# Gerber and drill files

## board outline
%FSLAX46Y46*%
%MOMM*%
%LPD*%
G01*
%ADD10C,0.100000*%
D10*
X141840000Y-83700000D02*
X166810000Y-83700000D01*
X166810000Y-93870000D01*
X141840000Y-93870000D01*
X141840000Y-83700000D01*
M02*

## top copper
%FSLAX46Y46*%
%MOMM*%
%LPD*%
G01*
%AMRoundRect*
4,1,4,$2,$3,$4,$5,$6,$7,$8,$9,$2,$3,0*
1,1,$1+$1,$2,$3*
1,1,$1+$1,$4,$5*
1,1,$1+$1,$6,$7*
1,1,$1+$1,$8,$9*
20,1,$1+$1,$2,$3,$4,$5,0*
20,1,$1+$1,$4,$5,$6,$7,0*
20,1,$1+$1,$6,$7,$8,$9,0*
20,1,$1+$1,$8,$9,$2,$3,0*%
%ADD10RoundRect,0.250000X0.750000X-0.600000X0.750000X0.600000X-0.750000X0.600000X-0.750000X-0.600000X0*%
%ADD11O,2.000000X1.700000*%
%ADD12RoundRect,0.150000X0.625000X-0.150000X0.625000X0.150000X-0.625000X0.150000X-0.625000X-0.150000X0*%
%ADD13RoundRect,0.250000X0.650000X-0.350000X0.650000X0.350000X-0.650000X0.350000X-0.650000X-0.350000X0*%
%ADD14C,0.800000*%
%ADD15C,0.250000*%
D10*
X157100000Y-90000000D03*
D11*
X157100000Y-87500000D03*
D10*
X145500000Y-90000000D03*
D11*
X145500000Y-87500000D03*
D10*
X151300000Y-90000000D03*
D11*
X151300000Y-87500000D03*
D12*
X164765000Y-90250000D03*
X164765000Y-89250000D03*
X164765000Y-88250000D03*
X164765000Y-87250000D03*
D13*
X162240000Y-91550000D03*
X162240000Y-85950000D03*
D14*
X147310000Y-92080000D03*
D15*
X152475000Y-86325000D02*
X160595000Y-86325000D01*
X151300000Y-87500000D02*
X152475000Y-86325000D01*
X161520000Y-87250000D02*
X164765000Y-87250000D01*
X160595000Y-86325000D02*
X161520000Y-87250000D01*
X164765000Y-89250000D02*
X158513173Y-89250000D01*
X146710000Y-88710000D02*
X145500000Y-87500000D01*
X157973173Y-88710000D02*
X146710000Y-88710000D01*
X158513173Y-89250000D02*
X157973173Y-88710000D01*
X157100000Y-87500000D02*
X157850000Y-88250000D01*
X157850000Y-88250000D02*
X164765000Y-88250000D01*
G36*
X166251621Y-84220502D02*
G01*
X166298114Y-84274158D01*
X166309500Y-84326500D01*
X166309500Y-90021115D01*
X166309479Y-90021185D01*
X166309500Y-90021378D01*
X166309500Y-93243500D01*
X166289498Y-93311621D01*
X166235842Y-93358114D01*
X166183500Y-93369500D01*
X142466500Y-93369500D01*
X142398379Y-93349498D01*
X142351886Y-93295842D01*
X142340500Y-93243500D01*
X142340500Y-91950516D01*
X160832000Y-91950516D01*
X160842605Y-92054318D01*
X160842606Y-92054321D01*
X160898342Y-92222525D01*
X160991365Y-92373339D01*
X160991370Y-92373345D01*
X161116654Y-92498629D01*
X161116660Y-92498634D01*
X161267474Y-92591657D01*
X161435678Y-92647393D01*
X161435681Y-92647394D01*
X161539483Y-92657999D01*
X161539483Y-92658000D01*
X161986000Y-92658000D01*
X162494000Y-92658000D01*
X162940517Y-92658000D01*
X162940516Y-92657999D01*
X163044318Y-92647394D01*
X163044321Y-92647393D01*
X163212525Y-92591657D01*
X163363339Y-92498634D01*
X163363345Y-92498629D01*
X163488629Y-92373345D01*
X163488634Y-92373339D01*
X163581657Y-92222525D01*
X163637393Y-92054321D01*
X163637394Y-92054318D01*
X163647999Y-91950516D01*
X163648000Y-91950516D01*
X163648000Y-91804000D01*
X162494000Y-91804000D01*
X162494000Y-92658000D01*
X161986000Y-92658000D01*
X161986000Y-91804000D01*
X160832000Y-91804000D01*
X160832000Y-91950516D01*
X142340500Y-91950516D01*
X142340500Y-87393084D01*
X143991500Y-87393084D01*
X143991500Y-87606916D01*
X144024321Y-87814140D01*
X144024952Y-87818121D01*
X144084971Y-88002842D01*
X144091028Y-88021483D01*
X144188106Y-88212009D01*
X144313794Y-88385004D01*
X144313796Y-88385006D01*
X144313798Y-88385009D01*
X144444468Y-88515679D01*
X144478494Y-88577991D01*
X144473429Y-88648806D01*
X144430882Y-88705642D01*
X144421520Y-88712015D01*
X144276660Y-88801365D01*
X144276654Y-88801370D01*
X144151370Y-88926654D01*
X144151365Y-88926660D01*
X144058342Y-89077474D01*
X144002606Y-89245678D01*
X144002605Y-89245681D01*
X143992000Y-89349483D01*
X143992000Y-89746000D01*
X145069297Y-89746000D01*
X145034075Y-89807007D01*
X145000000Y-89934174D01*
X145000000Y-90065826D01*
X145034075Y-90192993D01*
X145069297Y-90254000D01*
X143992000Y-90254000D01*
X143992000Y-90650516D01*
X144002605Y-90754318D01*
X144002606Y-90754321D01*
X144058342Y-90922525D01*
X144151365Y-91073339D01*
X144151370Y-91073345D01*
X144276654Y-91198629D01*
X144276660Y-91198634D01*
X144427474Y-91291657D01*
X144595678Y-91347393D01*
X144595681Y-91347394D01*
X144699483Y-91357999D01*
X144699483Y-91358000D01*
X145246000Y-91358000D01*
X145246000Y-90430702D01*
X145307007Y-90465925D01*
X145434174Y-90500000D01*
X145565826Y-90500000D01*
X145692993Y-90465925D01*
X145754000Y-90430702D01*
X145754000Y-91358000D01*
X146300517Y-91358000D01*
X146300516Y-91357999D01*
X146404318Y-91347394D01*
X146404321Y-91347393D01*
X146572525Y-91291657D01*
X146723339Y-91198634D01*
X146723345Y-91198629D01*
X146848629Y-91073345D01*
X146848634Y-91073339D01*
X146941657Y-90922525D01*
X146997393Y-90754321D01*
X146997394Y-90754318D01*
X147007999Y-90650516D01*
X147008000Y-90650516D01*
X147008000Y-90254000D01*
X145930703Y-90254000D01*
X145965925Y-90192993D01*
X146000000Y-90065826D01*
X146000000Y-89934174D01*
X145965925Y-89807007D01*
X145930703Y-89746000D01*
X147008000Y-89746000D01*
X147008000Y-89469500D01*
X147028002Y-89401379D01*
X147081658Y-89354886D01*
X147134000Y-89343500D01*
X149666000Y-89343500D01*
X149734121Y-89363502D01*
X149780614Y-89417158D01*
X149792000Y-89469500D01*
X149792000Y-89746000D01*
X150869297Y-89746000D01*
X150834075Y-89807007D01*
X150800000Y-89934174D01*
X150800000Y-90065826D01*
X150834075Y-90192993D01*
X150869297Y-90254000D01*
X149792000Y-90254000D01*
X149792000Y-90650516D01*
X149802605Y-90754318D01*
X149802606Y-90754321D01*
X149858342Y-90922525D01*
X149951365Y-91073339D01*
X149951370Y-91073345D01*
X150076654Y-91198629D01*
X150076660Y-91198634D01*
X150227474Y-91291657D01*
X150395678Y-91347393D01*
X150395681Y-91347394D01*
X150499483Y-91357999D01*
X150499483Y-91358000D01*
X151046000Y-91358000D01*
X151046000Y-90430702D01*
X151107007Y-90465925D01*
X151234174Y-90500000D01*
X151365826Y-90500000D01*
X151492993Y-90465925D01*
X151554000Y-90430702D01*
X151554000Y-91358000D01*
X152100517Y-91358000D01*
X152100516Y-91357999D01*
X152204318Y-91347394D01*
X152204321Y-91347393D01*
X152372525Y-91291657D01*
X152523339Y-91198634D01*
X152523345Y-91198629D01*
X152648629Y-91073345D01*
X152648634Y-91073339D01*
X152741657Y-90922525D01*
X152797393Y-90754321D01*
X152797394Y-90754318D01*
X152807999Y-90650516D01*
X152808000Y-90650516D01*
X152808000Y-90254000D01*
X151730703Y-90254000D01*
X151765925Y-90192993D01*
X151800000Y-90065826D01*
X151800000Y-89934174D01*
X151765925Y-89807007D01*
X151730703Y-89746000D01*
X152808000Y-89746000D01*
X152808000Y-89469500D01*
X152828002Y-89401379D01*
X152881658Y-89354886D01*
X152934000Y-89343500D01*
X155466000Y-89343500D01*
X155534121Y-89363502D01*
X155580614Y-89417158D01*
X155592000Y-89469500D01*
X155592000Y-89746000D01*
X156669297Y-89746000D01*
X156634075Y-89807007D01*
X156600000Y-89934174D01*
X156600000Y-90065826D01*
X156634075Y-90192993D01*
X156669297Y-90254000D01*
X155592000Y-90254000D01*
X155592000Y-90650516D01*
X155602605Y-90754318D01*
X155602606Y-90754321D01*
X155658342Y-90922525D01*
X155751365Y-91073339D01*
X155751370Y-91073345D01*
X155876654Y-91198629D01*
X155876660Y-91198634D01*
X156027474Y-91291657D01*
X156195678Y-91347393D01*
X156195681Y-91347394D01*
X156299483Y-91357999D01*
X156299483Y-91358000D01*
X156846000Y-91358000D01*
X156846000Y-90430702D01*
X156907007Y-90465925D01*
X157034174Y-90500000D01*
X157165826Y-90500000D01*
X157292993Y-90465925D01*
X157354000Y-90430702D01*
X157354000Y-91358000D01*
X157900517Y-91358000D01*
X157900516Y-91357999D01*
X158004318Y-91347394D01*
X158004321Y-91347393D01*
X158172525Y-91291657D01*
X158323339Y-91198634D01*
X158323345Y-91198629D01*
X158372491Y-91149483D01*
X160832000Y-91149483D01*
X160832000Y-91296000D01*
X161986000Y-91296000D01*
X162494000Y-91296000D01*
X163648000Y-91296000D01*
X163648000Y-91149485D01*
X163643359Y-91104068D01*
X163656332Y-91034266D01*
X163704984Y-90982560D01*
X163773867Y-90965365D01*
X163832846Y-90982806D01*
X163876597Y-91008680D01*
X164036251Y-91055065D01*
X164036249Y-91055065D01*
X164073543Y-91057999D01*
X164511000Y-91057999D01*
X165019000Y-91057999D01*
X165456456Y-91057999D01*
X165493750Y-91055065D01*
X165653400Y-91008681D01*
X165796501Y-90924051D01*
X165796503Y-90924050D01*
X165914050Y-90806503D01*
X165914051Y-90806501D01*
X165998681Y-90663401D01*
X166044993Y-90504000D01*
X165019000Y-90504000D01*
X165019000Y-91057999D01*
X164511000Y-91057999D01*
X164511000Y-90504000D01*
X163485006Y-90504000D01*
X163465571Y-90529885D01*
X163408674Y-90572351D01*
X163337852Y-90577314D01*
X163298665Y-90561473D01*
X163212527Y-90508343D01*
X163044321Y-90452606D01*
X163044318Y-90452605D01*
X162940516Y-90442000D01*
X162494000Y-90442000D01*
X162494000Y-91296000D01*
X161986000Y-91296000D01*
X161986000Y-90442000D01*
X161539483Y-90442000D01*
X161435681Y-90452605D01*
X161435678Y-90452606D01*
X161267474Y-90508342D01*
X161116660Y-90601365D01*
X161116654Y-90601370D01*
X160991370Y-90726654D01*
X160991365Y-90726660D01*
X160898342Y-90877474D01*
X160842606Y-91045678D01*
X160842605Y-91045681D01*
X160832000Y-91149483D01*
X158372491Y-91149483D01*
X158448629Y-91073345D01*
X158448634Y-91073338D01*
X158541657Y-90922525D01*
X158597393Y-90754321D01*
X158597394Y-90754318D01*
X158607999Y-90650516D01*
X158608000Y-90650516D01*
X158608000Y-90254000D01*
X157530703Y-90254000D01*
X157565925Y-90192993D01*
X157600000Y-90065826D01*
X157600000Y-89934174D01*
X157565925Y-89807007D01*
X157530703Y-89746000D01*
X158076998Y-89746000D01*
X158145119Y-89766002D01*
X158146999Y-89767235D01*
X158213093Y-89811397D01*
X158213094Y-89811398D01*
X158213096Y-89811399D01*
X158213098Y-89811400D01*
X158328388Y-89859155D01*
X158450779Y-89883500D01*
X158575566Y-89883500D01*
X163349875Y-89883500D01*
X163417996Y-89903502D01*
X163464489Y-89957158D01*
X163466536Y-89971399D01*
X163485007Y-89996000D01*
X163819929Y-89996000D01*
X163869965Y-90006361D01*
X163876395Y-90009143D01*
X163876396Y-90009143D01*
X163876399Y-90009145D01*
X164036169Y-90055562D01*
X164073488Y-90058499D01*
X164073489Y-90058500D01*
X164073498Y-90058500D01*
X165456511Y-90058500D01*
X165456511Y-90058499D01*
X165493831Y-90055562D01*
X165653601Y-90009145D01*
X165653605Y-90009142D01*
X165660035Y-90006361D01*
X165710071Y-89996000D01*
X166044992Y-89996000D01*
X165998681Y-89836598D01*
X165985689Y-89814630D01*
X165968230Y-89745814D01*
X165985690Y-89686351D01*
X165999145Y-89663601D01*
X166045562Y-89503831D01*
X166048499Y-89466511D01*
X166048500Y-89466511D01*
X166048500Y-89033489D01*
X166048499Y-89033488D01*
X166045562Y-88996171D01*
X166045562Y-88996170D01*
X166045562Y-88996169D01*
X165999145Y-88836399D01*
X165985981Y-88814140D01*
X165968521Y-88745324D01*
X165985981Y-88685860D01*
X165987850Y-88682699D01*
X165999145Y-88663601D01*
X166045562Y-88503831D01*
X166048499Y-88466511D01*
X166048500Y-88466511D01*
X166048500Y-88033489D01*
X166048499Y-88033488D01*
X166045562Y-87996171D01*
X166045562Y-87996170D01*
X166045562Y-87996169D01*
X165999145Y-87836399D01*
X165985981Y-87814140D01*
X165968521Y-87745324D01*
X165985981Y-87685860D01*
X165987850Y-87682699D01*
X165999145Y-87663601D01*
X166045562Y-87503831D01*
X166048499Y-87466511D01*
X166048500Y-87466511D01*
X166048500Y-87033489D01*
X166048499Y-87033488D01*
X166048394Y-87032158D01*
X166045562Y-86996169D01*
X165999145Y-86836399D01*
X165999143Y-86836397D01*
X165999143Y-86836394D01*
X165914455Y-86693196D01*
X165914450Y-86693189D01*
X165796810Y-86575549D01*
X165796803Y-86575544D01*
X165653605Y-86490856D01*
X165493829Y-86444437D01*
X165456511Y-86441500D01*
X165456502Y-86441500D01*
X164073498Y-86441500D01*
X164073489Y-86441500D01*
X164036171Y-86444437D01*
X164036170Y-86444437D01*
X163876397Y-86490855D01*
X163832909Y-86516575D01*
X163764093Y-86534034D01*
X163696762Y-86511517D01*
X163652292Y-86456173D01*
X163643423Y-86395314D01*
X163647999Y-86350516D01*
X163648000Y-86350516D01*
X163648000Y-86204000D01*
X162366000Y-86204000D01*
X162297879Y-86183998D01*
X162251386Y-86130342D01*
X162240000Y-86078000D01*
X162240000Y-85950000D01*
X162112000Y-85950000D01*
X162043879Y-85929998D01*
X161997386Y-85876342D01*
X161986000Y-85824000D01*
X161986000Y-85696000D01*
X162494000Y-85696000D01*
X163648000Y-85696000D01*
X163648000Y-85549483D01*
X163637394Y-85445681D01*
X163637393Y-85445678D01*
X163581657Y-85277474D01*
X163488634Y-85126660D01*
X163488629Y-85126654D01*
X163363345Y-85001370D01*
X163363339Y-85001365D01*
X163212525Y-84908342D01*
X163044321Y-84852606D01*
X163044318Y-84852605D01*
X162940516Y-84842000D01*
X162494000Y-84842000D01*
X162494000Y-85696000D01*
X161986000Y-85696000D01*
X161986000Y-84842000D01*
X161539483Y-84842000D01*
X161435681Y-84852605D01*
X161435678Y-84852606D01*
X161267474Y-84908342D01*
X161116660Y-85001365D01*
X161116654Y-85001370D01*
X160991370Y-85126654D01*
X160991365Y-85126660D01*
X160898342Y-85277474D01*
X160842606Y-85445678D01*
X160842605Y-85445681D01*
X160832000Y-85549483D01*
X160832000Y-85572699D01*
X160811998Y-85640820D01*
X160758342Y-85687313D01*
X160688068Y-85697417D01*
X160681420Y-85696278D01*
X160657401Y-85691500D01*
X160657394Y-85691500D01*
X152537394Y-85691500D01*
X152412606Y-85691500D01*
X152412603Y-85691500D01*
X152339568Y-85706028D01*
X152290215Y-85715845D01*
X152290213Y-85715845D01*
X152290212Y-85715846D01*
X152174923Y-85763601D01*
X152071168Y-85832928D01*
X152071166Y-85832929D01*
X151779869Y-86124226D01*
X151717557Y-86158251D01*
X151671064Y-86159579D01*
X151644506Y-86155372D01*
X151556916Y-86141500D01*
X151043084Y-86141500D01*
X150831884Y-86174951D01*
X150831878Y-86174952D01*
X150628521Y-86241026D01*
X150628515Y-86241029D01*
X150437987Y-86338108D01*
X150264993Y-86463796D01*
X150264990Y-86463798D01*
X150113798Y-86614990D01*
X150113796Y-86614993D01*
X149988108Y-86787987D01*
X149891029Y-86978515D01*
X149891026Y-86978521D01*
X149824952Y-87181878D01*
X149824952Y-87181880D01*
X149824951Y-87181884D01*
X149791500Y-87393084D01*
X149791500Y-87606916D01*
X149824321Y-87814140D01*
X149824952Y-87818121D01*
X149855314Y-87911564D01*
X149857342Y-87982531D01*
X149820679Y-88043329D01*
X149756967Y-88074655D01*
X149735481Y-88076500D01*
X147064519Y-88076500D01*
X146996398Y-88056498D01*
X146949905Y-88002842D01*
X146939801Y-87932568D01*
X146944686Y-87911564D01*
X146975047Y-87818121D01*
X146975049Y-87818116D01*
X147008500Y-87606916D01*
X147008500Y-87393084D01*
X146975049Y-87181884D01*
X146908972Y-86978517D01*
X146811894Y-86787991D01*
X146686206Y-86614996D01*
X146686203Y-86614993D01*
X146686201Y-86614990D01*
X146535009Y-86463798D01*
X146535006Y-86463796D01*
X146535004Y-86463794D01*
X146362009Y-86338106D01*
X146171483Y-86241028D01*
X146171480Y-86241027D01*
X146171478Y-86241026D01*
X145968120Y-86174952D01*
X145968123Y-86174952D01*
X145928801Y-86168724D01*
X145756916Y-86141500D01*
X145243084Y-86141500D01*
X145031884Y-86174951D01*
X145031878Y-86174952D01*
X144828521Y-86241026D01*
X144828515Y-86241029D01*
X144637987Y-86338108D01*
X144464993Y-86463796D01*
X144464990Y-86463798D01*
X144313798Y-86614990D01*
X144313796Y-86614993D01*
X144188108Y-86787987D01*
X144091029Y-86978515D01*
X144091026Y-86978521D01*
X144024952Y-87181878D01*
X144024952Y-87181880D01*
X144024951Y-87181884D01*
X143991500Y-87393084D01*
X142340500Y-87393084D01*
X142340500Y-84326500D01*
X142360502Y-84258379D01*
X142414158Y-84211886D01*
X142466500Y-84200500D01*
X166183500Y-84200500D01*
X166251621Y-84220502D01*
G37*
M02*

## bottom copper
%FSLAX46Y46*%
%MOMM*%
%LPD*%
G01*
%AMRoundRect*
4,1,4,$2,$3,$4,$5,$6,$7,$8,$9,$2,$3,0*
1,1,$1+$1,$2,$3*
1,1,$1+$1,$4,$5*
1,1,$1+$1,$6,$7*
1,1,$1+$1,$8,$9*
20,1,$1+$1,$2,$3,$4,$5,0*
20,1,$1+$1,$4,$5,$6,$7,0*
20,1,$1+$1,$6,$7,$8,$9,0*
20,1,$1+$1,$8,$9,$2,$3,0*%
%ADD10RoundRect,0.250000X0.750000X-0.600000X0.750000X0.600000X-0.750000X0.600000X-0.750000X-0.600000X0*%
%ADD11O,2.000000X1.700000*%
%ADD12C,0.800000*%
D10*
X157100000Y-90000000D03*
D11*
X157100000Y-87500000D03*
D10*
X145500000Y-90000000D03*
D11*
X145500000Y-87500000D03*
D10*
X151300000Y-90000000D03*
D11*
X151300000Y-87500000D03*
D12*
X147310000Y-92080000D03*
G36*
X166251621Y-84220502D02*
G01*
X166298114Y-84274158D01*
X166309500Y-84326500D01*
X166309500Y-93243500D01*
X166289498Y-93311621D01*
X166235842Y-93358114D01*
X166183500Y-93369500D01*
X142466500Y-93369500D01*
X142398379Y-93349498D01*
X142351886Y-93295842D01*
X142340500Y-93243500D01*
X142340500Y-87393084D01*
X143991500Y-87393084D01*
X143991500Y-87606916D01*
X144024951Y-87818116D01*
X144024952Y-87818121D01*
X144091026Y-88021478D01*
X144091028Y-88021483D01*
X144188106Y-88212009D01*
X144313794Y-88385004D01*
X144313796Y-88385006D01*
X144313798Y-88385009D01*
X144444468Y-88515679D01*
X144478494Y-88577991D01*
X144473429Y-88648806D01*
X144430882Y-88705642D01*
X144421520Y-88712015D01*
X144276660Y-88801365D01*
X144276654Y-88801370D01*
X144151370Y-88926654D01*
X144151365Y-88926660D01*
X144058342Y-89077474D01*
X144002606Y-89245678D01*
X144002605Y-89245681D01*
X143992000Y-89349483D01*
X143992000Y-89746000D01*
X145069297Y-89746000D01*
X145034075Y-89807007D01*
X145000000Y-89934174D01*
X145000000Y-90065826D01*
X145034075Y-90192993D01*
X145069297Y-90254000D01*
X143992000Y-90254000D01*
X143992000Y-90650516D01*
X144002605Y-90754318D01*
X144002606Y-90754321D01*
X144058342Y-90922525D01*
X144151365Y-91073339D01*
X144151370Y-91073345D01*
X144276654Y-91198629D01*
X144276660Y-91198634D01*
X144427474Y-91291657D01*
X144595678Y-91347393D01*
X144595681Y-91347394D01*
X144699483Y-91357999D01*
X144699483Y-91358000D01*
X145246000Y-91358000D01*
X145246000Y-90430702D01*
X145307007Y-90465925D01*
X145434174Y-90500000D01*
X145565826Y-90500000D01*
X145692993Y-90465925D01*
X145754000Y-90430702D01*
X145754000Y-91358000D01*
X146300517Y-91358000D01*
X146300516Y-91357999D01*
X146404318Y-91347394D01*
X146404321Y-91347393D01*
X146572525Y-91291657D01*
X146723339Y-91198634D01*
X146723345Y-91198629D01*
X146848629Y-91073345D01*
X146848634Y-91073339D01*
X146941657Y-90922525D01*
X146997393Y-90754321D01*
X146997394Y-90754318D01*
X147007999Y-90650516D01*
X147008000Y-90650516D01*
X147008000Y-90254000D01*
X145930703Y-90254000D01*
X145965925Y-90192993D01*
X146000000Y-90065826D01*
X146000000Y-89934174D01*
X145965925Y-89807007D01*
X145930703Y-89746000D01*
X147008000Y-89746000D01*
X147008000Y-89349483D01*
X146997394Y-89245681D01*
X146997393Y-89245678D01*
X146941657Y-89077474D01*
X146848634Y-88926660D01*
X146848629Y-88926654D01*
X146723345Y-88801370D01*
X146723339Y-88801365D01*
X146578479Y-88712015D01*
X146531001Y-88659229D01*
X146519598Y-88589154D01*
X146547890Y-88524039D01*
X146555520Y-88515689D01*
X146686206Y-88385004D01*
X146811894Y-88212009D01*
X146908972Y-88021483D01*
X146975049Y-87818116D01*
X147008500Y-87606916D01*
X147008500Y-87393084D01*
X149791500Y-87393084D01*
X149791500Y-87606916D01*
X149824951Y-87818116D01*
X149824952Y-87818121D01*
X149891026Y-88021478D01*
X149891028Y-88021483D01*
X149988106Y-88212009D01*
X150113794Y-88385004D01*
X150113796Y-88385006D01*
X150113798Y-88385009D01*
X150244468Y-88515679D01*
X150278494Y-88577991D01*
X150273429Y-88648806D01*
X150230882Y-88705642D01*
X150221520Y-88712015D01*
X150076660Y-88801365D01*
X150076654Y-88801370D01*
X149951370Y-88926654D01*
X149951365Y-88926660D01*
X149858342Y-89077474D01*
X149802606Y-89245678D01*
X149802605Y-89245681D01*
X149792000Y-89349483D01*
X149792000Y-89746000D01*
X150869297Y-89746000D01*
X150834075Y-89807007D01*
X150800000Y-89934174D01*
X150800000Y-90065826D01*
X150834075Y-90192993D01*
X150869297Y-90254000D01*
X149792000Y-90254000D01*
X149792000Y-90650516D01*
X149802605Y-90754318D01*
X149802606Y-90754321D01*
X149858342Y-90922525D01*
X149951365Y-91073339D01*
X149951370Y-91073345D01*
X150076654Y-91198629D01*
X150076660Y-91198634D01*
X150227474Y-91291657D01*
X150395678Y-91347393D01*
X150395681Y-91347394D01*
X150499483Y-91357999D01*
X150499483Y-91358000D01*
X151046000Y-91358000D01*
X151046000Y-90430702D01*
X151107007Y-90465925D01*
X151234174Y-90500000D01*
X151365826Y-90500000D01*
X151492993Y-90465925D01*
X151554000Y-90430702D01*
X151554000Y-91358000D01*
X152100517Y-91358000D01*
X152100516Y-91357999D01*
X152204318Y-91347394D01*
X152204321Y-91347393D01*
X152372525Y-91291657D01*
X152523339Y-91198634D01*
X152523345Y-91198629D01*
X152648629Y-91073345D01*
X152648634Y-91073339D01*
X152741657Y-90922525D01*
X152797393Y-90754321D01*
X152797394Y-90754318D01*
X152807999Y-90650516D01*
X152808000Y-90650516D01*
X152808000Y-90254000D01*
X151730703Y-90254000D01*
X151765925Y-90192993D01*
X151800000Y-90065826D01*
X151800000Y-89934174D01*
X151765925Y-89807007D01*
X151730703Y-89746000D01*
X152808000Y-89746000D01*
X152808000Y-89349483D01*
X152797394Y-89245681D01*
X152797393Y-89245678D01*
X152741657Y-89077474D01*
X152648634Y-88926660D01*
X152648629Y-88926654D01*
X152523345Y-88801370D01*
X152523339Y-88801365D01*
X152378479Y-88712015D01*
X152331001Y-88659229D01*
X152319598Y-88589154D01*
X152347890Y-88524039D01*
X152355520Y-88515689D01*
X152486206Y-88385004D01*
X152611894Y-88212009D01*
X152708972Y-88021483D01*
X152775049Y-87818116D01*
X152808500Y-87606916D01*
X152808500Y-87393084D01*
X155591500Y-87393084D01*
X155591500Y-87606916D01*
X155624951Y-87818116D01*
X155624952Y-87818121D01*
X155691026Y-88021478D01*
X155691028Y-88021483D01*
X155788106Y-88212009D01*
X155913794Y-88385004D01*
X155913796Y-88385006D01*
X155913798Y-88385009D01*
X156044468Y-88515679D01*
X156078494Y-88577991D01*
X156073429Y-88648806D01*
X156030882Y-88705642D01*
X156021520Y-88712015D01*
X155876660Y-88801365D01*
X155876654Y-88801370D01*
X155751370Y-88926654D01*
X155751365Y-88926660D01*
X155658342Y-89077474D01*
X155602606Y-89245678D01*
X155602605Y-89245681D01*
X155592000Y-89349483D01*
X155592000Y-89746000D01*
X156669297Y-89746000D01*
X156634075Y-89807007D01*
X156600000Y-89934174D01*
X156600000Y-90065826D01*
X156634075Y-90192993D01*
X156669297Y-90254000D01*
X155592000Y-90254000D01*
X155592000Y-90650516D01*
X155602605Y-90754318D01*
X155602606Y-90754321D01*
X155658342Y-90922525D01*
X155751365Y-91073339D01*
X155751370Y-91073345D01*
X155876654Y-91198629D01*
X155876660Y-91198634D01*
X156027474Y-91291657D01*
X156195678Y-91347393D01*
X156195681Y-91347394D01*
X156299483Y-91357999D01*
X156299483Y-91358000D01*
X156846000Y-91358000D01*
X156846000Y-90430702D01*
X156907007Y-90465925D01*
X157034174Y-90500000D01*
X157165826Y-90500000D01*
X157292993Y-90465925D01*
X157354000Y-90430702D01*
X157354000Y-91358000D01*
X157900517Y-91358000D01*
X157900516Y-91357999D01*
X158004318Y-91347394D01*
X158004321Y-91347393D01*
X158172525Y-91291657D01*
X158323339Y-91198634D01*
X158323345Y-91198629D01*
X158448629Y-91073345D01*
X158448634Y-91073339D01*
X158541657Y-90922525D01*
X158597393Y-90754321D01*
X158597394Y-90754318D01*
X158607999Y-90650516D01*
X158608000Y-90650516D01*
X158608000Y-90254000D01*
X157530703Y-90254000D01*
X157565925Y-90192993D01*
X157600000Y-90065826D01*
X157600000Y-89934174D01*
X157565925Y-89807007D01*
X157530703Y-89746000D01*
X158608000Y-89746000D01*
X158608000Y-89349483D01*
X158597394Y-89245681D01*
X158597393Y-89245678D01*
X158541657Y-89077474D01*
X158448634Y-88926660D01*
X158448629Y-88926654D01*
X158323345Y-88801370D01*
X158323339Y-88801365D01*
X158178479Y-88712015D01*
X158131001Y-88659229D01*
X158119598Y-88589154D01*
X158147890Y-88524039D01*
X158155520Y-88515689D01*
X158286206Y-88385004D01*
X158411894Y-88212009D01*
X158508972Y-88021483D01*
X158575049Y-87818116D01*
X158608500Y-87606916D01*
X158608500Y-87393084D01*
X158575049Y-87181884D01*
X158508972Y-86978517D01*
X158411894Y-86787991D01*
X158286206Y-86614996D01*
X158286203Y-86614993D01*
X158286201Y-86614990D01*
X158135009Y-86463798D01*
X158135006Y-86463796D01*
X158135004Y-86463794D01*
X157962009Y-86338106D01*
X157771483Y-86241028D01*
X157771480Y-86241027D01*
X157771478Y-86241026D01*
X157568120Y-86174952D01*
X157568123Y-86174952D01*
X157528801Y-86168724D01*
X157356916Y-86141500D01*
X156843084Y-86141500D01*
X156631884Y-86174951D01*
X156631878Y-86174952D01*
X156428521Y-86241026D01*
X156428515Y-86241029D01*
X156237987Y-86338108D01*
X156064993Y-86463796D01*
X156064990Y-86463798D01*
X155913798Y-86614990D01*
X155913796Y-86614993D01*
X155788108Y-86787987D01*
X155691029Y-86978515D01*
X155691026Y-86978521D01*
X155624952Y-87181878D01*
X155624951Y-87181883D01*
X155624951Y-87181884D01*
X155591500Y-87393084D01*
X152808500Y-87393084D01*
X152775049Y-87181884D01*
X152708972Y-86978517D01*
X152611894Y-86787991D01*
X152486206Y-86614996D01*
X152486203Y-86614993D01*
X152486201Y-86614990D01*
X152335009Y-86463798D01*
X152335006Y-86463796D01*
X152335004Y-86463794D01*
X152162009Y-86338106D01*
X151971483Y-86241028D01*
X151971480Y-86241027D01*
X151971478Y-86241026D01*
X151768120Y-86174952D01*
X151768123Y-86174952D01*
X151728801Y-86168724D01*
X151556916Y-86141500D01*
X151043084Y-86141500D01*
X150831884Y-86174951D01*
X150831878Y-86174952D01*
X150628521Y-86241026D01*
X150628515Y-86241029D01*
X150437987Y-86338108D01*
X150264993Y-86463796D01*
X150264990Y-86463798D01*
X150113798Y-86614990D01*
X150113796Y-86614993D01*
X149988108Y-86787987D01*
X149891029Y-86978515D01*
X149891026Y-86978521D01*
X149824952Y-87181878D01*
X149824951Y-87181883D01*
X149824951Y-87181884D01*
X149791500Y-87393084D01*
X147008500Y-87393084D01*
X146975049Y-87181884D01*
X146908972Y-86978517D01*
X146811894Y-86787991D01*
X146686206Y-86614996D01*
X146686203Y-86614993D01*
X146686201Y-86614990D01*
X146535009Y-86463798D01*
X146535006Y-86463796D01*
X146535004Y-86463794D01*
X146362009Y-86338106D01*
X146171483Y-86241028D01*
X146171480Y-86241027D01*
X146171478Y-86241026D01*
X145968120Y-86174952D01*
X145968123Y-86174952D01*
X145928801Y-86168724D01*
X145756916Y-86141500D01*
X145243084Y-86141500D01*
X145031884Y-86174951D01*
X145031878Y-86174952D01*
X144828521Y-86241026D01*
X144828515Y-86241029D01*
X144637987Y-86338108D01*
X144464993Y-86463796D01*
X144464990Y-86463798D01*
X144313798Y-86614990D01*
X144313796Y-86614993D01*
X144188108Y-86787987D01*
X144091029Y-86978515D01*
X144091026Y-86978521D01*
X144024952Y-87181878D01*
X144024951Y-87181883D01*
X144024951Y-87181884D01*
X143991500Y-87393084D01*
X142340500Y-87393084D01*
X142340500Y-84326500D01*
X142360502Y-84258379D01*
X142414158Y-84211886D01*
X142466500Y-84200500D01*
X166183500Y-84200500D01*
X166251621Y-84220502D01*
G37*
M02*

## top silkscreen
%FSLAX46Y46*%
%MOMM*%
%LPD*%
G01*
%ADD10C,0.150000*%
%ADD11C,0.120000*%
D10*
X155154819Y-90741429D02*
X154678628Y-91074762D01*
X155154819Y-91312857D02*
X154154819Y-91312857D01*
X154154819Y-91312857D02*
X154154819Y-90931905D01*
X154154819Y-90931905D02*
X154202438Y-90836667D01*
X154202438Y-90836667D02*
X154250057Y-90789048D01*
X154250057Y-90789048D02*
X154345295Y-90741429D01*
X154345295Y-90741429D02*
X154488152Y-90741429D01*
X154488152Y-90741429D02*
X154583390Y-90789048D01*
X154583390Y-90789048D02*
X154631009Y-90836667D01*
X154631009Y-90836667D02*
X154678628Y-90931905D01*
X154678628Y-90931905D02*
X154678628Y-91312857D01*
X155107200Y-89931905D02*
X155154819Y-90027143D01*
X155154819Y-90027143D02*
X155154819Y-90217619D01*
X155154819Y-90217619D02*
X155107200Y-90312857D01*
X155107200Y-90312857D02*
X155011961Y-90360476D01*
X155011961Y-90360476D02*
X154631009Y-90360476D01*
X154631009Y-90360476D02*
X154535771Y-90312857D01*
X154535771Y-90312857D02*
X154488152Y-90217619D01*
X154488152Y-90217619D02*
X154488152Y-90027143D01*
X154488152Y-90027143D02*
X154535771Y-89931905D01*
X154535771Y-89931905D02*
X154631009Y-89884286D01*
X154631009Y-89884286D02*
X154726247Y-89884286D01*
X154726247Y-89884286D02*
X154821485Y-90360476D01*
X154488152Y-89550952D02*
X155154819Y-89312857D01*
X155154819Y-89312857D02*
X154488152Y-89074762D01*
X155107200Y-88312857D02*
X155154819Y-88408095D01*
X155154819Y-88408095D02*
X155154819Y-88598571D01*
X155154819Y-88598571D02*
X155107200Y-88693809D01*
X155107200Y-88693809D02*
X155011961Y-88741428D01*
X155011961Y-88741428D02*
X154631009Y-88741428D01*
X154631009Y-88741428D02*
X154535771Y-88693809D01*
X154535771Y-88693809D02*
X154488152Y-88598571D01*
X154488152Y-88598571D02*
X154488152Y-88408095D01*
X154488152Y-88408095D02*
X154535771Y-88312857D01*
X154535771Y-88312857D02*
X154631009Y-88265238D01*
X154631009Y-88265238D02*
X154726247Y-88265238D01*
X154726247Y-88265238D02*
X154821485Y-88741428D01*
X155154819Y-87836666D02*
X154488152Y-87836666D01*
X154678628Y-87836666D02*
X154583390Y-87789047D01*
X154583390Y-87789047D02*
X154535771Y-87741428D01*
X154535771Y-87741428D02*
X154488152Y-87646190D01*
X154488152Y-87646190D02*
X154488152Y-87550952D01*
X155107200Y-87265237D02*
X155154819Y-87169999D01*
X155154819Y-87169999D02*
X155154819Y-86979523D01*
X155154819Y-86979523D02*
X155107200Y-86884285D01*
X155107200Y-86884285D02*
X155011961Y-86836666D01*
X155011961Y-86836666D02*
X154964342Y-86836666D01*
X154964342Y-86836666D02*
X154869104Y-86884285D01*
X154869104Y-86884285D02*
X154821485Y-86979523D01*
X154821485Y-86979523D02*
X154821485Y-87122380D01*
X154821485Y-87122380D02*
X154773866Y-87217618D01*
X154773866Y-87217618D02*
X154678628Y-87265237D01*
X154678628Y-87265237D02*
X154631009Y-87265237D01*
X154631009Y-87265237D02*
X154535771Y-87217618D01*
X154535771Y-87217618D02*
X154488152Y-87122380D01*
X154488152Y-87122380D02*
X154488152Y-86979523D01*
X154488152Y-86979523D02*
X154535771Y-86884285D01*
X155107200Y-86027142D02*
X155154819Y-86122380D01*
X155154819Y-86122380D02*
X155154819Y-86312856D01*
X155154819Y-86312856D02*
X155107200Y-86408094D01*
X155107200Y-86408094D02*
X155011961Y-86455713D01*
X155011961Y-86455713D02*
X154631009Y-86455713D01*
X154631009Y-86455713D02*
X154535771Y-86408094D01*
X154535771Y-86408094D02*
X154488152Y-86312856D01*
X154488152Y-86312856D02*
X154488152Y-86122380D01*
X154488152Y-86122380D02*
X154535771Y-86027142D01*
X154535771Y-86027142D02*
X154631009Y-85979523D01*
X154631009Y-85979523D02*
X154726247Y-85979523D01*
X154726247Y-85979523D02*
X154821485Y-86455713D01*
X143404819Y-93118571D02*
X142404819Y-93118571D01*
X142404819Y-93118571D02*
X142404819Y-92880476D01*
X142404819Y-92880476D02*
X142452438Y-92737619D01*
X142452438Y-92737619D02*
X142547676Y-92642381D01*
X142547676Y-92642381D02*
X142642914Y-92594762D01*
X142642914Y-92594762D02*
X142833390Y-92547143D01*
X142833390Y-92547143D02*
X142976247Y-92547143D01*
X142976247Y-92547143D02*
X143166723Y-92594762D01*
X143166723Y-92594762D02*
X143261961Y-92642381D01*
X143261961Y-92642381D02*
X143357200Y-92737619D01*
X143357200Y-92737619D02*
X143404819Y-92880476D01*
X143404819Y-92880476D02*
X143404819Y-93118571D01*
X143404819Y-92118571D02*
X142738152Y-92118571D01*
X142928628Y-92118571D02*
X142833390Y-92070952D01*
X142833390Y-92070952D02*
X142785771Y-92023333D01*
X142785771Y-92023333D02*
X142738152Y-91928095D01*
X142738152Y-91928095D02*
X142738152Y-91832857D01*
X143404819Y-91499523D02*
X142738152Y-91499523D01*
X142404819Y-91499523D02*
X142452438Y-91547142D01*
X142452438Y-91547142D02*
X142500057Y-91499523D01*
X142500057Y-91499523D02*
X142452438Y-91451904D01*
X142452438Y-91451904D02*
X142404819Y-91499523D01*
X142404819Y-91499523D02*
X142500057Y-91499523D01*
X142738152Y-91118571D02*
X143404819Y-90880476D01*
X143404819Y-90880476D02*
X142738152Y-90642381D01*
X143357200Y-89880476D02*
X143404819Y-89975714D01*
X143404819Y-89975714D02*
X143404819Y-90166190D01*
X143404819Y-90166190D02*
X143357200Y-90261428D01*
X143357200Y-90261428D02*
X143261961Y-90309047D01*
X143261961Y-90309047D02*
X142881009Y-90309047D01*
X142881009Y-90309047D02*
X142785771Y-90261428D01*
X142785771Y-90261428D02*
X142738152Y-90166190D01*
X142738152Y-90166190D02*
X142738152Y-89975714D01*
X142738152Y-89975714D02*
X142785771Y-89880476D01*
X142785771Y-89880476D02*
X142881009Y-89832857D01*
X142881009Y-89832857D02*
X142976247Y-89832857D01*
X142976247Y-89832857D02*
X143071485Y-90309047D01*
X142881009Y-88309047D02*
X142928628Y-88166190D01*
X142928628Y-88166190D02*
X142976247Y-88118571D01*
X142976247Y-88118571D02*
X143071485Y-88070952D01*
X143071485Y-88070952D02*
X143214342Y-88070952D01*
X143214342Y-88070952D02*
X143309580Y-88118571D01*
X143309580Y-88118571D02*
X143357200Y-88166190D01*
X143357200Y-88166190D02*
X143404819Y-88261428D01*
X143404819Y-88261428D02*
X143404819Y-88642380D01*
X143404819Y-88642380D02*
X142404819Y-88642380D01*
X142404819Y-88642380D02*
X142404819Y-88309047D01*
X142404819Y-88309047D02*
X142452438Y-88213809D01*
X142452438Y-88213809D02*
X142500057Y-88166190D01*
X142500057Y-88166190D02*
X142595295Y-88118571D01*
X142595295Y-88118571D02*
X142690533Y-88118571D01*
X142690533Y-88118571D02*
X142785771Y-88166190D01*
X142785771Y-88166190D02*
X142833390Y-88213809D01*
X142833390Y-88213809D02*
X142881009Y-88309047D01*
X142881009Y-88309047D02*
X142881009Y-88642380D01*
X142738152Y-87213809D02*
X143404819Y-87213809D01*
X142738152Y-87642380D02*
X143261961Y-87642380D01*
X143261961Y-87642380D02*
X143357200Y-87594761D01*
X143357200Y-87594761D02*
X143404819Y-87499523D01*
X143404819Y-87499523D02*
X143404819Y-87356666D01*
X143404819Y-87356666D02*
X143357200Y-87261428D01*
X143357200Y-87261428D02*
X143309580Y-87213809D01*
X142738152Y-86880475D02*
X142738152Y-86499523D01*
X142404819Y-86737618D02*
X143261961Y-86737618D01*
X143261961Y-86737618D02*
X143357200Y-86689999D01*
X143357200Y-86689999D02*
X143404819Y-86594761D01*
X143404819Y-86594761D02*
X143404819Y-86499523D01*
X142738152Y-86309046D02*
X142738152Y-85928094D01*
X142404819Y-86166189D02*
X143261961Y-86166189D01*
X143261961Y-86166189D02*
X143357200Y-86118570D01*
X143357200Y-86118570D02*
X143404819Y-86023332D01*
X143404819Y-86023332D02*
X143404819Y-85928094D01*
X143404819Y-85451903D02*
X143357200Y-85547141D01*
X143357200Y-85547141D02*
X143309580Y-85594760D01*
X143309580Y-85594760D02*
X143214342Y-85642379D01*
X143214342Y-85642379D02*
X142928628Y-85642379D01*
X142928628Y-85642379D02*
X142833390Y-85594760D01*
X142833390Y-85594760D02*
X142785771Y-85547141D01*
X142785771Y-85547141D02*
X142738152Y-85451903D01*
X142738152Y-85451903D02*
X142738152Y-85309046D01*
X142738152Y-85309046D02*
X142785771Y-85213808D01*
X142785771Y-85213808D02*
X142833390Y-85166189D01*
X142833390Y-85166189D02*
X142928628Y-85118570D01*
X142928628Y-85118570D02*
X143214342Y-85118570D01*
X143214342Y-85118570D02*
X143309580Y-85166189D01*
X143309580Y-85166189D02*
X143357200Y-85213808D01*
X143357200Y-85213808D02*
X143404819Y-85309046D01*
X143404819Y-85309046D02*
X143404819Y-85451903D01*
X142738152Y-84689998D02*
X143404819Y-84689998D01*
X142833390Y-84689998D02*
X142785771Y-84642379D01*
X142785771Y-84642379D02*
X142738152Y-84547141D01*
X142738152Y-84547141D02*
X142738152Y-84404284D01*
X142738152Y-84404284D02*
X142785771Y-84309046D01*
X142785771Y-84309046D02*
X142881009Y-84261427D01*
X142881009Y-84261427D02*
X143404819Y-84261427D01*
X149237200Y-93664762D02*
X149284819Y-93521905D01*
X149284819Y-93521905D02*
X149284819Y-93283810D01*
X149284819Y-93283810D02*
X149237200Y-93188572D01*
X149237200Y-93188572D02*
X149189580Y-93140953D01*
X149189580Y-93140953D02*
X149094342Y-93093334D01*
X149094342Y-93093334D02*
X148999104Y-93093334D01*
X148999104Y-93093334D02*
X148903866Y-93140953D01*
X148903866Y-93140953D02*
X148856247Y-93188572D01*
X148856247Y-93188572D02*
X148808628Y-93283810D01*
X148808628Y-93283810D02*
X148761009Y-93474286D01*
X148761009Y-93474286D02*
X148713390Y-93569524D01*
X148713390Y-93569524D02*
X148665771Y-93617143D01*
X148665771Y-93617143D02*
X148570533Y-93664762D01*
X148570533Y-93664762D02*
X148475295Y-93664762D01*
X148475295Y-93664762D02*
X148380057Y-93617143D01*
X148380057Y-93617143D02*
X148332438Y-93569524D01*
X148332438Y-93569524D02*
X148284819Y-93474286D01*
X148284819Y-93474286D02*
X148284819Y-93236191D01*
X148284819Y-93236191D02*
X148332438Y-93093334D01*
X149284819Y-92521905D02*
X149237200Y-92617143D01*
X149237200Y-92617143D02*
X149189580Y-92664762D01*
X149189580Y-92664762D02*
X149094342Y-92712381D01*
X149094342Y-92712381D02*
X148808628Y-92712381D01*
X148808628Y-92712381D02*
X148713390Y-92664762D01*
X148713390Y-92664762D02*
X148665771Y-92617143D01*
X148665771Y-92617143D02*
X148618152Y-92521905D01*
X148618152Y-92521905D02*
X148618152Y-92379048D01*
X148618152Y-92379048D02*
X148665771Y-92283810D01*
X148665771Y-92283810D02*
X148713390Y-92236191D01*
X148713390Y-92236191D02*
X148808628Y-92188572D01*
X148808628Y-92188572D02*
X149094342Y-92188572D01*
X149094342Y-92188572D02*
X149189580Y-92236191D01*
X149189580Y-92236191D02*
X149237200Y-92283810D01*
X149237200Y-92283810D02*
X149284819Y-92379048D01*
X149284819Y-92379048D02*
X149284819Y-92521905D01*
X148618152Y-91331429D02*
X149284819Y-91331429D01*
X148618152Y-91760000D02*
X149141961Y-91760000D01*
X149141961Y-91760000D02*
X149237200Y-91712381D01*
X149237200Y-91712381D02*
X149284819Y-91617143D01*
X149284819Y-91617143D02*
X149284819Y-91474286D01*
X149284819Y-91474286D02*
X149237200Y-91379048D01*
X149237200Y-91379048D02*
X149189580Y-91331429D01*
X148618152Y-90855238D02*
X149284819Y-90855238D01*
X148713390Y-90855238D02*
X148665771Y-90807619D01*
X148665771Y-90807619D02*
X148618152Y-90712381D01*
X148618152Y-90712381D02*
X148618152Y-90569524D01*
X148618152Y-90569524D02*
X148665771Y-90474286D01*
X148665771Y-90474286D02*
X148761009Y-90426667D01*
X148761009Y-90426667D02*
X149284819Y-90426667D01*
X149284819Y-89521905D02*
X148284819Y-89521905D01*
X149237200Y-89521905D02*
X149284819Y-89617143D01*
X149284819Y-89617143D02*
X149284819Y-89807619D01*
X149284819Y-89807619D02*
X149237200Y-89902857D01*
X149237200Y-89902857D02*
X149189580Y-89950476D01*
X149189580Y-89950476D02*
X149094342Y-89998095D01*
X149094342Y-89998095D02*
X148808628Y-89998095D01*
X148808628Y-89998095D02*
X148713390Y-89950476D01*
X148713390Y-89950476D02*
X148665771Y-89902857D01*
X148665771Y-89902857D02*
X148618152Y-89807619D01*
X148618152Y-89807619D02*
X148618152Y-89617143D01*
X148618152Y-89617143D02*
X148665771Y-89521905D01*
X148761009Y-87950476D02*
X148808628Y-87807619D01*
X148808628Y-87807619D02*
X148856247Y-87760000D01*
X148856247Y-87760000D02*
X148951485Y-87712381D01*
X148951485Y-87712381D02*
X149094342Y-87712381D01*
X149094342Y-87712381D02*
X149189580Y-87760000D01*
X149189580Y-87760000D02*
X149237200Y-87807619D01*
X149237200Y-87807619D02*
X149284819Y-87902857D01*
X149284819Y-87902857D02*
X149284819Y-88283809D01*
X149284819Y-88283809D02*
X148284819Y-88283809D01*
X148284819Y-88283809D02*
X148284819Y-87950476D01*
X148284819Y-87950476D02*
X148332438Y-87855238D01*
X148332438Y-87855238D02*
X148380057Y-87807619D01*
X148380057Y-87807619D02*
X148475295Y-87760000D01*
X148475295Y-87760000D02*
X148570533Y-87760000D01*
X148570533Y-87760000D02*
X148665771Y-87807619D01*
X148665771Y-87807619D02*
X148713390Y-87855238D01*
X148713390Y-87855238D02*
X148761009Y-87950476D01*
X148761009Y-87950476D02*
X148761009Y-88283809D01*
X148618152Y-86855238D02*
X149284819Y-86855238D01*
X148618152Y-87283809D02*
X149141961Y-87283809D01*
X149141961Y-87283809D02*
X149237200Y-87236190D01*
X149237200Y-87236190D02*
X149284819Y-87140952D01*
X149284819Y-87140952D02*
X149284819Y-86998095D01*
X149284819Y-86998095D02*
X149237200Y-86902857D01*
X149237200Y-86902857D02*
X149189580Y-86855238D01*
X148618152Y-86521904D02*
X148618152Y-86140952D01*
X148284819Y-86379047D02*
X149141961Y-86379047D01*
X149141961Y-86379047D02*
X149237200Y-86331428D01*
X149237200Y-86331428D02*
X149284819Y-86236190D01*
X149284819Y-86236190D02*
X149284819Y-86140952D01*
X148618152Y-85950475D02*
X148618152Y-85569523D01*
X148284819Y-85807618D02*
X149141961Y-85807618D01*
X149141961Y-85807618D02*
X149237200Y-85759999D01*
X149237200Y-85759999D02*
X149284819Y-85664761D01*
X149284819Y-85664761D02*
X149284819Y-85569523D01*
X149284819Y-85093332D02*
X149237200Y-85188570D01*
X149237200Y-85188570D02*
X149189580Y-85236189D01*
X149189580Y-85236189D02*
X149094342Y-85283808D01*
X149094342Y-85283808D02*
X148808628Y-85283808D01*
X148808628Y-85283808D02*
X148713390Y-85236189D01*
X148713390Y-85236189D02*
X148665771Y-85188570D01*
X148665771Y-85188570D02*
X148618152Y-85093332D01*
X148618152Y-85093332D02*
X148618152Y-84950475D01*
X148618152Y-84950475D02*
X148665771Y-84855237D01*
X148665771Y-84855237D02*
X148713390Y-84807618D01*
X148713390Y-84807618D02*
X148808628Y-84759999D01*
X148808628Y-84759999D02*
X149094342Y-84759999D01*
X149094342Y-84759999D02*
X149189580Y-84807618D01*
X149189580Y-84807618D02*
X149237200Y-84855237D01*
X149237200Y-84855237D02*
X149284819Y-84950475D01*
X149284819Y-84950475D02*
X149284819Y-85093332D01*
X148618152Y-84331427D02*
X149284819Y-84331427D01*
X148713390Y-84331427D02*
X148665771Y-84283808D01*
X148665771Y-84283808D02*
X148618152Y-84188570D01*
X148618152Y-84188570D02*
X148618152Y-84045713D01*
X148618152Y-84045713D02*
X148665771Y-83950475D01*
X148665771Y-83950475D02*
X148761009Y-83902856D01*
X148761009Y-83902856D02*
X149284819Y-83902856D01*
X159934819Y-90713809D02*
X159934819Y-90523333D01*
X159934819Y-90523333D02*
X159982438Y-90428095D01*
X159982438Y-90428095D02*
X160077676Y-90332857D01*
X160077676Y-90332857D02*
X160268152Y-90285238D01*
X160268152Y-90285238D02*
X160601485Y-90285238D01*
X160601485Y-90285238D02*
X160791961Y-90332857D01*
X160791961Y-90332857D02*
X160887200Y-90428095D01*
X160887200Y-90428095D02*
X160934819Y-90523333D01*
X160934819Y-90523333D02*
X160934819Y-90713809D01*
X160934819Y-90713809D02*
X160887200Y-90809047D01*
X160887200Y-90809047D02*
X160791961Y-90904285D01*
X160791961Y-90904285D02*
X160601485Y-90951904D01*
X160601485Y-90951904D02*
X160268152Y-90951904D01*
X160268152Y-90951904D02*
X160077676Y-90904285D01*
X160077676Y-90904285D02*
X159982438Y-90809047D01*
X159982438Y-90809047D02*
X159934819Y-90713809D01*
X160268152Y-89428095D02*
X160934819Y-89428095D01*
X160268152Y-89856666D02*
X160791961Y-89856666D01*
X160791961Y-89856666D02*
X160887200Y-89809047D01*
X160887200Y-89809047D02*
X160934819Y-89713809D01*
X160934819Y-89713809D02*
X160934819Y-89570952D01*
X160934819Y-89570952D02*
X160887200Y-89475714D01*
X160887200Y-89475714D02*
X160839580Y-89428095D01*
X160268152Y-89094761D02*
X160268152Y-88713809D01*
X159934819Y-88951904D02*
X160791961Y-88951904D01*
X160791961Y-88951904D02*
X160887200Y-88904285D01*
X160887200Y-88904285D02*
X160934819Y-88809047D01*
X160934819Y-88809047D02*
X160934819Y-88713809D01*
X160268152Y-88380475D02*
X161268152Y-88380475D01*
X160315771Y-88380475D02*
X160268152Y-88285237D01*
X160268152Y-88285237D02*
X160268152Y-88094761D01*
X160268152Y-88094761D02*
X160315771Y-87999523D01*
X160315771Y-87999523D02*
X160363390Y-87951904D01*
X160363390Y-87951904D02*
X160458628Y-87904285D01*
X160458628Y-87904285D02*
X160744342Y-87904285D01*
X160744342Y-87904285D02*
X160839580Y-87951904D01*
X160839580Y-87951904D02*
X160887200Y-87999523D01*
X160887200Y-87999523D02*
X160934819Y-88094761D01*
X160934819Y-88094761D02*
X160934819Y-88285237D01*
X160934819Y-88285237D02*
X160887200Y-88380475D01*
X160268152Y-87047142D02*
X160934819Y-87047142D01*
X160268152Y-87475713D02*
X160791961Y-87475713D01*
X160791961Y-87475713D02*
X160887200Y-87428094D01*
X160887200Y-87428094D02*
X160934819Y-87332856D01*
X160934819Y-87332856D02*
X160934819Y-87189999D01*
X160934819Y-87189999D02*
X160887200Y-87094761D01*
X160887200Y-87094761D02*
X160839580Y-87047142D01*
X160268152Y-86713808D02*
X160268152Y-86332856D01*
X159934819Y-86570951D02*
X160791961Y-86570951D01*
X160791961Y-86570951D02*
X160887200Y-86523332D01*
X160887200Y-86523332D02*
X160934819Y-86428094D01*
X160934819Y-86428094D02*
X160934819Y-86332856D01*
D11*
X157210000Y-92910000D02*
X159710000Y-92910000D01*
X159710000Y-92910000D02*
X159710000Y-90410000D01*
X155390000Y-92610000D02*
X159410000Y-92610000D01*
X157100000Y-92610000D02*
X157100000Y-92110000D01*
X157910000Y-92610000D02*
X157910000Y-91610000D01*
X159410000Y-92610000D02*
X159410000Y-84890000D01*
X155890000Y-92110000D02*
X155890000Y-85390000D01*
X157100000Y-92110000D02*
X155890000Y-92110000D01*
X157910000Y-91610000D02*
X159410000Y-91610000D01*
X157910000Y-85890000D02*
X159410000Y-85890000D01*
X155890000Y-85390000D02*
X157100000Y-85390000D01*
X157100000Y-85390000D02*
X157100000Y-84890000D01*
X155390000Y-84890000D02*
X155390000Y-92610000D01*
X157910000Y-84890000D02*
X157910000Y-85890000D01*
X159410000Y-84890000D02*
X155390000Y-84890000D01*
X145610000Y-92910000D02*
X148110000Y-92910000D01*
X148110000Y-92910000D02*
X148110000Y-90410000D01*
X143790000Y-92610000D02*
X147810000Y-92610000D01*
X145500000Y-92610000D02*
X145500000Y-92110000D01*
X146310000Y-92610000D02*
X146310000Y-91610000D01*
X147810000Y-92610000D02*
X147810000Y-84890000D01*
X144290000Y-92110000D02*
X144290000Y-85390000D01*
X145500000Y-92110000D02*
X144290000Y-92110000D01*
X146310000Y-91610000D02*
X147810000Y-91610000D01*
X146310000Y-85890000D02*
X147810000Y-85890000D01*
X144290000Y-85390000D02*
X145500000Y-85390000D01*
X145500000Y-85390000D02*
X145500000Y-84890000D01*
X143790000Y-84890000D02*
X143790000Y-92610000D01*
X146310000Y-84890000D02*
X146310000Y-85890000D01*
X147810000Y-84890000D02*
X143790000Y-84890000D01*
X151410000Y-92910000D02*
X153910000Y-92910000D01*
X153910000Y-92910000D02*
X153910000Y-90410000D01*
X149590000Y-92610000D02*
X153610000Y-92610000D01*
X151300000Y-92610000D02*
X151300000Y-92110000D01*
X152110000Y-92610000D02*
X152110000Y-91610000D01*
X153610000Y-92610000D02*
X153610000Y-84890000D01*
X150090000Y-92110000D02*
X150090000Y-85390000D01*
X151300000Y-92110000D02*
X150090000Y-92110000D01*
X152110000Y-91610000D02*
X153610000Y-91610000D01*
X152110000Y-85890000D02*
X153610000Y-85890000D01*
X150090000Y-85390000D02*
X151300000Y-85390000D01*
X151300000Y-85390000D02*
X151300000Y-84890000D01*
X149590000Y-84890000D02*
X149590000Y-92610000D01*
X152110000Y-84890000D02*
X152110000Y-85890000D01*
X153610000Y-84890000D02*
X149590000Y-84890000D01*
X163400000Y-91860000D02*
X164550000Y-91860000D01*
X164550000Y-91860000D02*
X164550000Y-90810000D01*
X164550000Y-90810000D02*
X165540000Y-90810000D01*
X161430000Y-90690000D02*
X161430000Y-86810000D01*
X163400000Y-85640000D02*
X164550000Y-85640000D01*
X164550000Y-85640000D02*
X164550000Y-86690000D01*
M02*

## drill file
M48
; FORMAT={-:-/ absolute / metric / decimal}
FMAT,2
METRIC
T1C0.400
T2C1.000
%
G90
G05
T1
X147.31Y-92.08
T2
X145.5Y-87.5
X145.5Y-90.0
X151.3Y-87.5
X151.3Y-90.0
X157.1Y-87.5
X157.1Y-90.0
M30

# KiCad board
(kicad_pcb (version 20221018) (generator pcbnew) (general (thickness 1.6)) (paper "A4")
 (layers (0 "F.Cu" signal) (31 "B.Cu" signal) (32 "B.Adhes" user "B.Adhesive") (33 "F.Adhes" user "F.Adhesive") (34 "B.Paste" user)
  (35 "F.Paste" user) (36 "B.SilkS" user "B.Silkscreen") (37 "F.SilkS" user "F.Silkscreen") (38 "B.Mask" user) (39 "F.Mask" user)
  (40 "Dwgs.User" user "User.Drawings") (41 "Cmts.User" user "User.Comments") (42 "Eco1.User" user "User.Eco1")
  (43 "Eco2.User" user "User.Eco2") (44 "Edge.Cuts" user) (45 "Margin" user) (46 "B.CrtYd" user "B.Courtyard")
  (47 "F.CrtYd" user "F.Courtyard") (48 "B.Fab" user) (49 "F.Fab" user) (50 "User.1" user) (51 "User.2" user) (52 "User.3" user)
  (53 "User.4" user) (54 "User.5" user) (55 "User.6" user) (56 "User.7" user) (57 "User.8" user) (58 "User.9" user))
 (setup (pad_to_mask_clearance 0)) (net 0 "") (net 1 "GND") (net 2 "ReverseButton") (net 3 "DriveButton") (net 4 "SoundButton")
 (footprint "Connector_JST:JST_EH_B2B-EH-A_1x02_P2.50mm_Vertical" (layer "F.Cu") (at 157.1 90 90)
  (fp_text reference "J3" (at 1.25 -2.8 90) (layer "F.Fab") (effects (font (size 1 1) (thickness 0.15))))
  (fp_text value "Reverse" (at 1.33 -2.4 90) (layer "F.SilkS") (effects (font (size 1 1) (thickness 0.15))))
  (fp_line (start -2.91 0.11) (end -2.91 2.61) (stroke (width 0.12) (type solid)) (layer "F.SilkS"))
  (fp_line (start -2.91 2.61) (end -0.41 2.61) (stroke (width 0.12) (type solid)) (layer "F.SilkS"))
  (fp_line (start -2.61 -1.71) (end -2.61 2.31) (stroke (width 0.12) (type solid)) (layer "F.SilkS"))
  (fp_line (start -2.61 0) (end -2.11 0) (stroke (width 0.12) (type solid)) (layer "F.SilkS"))
  (fp_line (start -2.61 0.81) (end -1.61 0.81) (stroke (width 0.12) (type solid)) (layer "F.SilkS"))
  (fp_line (start -2.61 2.31) (end 5.11 2.31) (stroke (width 0.12) (type solid)) (layer "F.SilkS"))
  (fp_line (start -2.11 -1.21) (end 4.61 -1.21) (stroke (width 0.12) (type solid)) (layer "F.SilkS"))
  (fp_line (start -2.11 0) (end -2.11 -1.21) (stroke (width 0.12) (type solid)) (layer "F.SilkS"))
  (fp_line (start -1.61 0.81) (end -1.61 2.31) (stroke (width 0.12) (type solid)) (layer "F.SilkS"))
  (fp_line (start 4.11 0.81) (end 4.11 2.31) (stroke (width 0.12) (type solid)) (layer "F.SilkS"))
  (fp_line (start 4.61 -1.21) (end 4.61 0) (stroke (width 0.12) (type solid)) (layer "F.SilkS"))
  (fp_line (start 4.61 0) (end 5.11 0) (stroke (width 0.12) (type solid)) (layer "F.SilkS"))
  (fp_line (start 5.11 -1.71) (end -2.61 -1.71) (stroke (width 0.12) (type solid)) (layer "F.SilkS"))
  (fp_line (start 5.11 0.81) (end 4.11 0.81) (stroke (width 0.12) (type solid)) (layer "F.SilkS"))
  (fp_line (start 5.11 2.31) (end 5.11 -1.71) (stroke (width 0.12) (type solid)) (layer "F.SilkS"))
  (pad "1" thru_hole roundrect (at 0 0 90) (size 1.7 2) (drill 1) (layers "*.Cu" "*.Mask") (roundrect_rratio 0.1470588235) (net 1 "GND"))
  (pad "2" thru_hole oval (at 2.5 0 90) (size 1.7 2) (drill 1) (layers "*.Cu" "*.Mask") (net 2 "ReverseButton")))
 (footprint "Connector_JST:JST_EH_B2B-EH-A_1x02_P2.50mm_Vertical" (layer "F.Cu") (at 145.5 90 90)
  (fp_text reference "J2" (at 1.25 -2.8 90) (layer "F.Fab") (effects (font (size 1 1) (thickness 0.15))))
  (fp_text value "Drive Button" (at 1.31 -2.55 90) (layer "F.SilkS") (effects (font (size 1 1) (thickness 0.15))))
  (fp_line (start -2.91 0.11) (end -2.91 2.61) (stroke (width 0.12) (type solid)) (layer "F.SilkS"))
  (fp_line (start -2.91 2.61) (end -0.41 2.61) (stroke (width 0.12) (type solid)) (layer "F.SilkS"))
  (fp_line (start -2.61 -1.71) (end -2.61 2.31) (stroke (width 0.12) (type solid)) (layer "F.SilkS"))
  (fp_line (start -2.61 0) (end -2.11 0) (stroke (width 0.12) (type solid)) (layer "F.SilkS"))
  (fp_line (start -2.61 0.81) (end -1.61 0.81) (stroke (width 0.12) (type solid)) (layer "F.SilkS"))
  (fp_line (start -2.61 2.31) (end 5.11 2.31) (stroke (width 0.12) (type solid)) (layer "F.SilkS"))
  (fp_line (start -2.11 -1.21) (end 4.61 -1.21) (stroke (width 0.12) (type solid)) (layer "F.SilkS"))
  (fp_line (start -2.11 0) (end -2.11 -1.21) (stroke (width 0.12) (type solid)) (layer "F.SilkS"))
  (fp_line (start -1.61 0.81) (end -1.61 2.31) (stroke (width 0.12) (type solid)) (layer "F.SilkS"))
  (fp_line (start 4.11 0.81) (end 4.11 2.31) (stroke (width 0.12) (type solid)) (layer "F.SilkS"))
  (fp_line (start 4.61 -1.21) (end 4.61 0) (stroke (width 0.12) (type solid)) (layer "F.SilkS"))
  (fp_line (start 4.61 0) (end 5.11 0) (stroke (width 0.12) (type solid)) (layer "F.SilkS"))
  (fp_line (start 5.11 -1.71) (end -2.61 -1.71) (stroke (width 0.12) (type solid)) (layer "F.SilkS"))
  (fp_line (start 5.11 0.81) (end 4.11 0.81) (stroke (width 0.12) (type solid)) (layer "F.SilkS"))
  (fp_line (start 5.11 2.31) (end 5.11 -1.71) (stroke (width 0.12) (type solid)) (layer "F.SilkS"))
  (pad "1" thru_hole roundrect (at 0 0 90) (size 1.7 2) (drill 1) (layers "*.Cu" "*.Mask") (roundrect_rratio 0.1470588235) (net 1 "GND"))
  (pad "2" thru_hole oval (at 2.5 0 90) (size 1.7 2) (drill 1) (layers "*.Cu" "*.Mask") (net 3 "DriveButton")))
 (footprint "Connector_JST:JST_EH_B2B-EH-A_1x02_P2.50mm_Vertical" (layer "F.Cu") (at 151.3 90 90)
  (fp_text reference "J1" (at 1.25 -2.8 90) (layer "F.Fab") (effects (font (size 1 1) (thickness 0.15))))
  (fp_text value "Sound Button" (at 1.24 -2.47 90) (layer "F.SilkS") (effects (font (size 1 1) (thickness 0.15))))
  (fp_line (start -2.91 0.11) (end -2.91 2.61) (stroke (width 0.12) (type solid)) (layer "F.SilkS"))
  (fp_line (start -2.91 2.61) (end -0.41 2.61) (stroke (width 0.12) (type solid)) (layer "F.SilkS"))
  (fp_line (start -2.61 -1.71) (end -2.61 2.31) (stroke (width 0.12) (type solid)) (layer "F.SilkS"))
  (fp_line (start -2.61 0) (end -2.11 0) (stroke (width 0.12) (type solid)) (layer "F.SilkS"))
  (fp_line (start -2.61 0.81) (end -1.61 0.81) (stroke (width 0.12) (type solid)) (layer "F.SilkS"))
  (fp_line (start -2.61 2.31) (end 5.11 2.31) (stroke (width 0.12) (type solid)) (layer "F.SilkS"))
  (fp_line (start -2.11 -1.21) (end 4.61 -1.21) (stroke (width 0.12) (type solid)) (layer "F.SilkS"))
  (fp_line (start -2.11 0) (end -2.11 -1.21) (stroke (width 0.12) (type solid)) (layer "F.SilkS"))
  (fp_line (start -1.61 0.81) (end -1.61 2.31) (stroke (width 0.12) (type solid)) (layer "F.SilkS"))
  (fp_line (start 4.11 0.81) (end 4.11 2.31) (stroke (width 0.12) (type solid)) (layer "F.SilkS"))
  (fp_line (start 4.61 -1.21) (end 4.61 0) (stroke (width 0.12) (type solid)) (layer "F.SilkS"))
  (fp_line (start 4.61 0) (end 5.11 0) (stroke (width 0.12) (type solid)) (layer "F.SilkS"))
  (fp_line (start 5.11 -1.71) (end -2.61 -1.71) (stroke (width 0.12) (type solid)) (layer "F.SilkS"))
  (fp_line (start 5.11 0.81) (end 4.11 0.81) (stroke (width 0.12) (type solid)) (layer "F.SilkS"))
  (fp_line (start 5.11 2.31) (end 5.11 -1.71) (stroke (width 0.12) (type solid)) (layer "F.SilkS"))
  (pad "1" thru_hole roundrect (at 0 0 90) (size 1.7 2) (drill 1) (layers "*.Cu" "*.Mask") (roundrect_rratio 0.1470588235) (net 1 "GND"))
  (pad "2" thru_hole oval (at 2.5 0 90) (size 1.7 2) (drill 1) (layers "*.Cu" "*.Mask") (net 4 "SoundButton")))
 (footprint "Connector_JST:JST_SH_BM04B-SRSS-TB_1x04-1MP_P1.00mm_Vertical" (layer "F.Cu") (at 163.44 88.75 90)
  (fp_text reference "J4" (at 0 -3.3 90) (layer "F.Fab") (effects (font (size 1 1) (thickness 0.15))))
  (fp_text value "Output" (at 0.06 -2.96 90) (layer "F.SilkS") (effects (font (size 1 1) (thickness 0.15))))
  (fp_line (start -3.11 -0.04) (end -3.11 1.11) (stroke (width 0.12) (type solid)) (layer "F.SilkS"))
  (fp_line (start -3.11 1.11) (end -2.06 1.11) (stroke (width 0.12) (type solid)) (layer "F.SilkS"))
  (fp_line (start -2.06 1.11) (end -2.06 2.1) (stroke (width 0.12) (type solid)) (layer "F.SilkS"))
  (fp_line (start -1.94 -2.01) (end 1.94 -2.01) (stroke (width 0.12) (type solid)) (layer "F.SilkS"))
  (fp_line (start 3.11 -0.04) (end 3.11 1.11) (stroke (width 0.12) (type solid)) (layer "F.SilkS"))
  (fp_line (start 3.11 1.11) (end 2.06 1.11) (stroke (width 0.12) (type solid)) (layer "F.SilkS"))
  (pad "1" smd roundrect (at -1.5 1.325 90) (size 0.6 1.55) (layers "F.Cu" "F.Paste" "F.Mask") (roundrect_rratio 0.25) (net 1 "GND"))
  (pad "2" smd roundrect (at -0.5 1.325 90) (size 0.6 1.55) (layers "F.Cu" "F.Paste" "F.Mask") (roundrect_rratio 0.25) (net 3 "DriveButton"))
  (pad "3" smd roundrect (at 0.5 1.325 90) (size 0.6 1.55) (layers "F.Cu" "F.Paste" "F.Mask") (roundrect_rratio 0.25)
   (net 2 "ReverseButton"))
  (pad "4" smd roundrect (at 1.5 1.325 90) (size 0.6 1.55) (layers "F.Cu" "F.Paste" "F.Mask") (roundrect_rratio 0.25) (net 4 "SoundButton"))
  (pad "MP" smd roundrect (at -2.8 -1.2 90) (size 1.2 1.8) (layers "F.Cu" "F.Paste" "F.Mask") (roundrect_rratio 0.2083333333) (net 1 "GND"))
  (pad "MP" smd roundrect (at 2.8 -1.2 90) (size 1.2 1.8) (layers "F.Cu" "F.Paste" "F.Mask") (roundrect_rratio 0.2083333333) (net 1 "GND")))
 (gr_rect (start 141.84 83.7) (end 166.81 93.87) (stroke (width 0.1) (type solid)) (fill none) (layer "Edge.Cuts"))
 (via (at 147.31 92.08) (size 0.8) (drill 0.4) (layers "F.Cu" "B.Cu") (free) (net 1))
 (segment (start 152.475 86.325) (end 160.595 86.325) (width 0.25) (layer "F.Cu") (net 4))
 (segment (start 151.3 87.5) (end 152.475 86.325) (width 0.25) (layer "F.Cu") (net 4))
 (segment (start 161.52 87.25) (end 164.765 87.25) (width 0.25) (layer "F.Cu") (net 4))
 (segment (start 160.595 86.325) (end 161.52 87.25) (width 0.25) (layer "F.Cu") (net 4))
 (segment (start 164.765 89.25) (end 158.513173 89.25) (width 0.25) (layer "F.Cu") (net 3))
 (segment (start 146.71 88.71) (end 145.5 87.5) (width 0.25) (layer "F.Cu") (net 3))
 (segment (start 157.973173 88.71) (end 146.71 88.71) (width 0.25) (layer "F.Cu") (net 3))
 (segment (start 158.513173 89.25) (end 157.973173 88.71) (width 0.25) (layer "F.Cu") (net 3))
 (segment (start 157.1 87.5) (end 157.85 88.25) (width 0.25) (layer "F.Cu") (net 2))
 (segment (start 157.85 88.25) (end 164.765 88.25) (width 0.25) (layer "F.Cu") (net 2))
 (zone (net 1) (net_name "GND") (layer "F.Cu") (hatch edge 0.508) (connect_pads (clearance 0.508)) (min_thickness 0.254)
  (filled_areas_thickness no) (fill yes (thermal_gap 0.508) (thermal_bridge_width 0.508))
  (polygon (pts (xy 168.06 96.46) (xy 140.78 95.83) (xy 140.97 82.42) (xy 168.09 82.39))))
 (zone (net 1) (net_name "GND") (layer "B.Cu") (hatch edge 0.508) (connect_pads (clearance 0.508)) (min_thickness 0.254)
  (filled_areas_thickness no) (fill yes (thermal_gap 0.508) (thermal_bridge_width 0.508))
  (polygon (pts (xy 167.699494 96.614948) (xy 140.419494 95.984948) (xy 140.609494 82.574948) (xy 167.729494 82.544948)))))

